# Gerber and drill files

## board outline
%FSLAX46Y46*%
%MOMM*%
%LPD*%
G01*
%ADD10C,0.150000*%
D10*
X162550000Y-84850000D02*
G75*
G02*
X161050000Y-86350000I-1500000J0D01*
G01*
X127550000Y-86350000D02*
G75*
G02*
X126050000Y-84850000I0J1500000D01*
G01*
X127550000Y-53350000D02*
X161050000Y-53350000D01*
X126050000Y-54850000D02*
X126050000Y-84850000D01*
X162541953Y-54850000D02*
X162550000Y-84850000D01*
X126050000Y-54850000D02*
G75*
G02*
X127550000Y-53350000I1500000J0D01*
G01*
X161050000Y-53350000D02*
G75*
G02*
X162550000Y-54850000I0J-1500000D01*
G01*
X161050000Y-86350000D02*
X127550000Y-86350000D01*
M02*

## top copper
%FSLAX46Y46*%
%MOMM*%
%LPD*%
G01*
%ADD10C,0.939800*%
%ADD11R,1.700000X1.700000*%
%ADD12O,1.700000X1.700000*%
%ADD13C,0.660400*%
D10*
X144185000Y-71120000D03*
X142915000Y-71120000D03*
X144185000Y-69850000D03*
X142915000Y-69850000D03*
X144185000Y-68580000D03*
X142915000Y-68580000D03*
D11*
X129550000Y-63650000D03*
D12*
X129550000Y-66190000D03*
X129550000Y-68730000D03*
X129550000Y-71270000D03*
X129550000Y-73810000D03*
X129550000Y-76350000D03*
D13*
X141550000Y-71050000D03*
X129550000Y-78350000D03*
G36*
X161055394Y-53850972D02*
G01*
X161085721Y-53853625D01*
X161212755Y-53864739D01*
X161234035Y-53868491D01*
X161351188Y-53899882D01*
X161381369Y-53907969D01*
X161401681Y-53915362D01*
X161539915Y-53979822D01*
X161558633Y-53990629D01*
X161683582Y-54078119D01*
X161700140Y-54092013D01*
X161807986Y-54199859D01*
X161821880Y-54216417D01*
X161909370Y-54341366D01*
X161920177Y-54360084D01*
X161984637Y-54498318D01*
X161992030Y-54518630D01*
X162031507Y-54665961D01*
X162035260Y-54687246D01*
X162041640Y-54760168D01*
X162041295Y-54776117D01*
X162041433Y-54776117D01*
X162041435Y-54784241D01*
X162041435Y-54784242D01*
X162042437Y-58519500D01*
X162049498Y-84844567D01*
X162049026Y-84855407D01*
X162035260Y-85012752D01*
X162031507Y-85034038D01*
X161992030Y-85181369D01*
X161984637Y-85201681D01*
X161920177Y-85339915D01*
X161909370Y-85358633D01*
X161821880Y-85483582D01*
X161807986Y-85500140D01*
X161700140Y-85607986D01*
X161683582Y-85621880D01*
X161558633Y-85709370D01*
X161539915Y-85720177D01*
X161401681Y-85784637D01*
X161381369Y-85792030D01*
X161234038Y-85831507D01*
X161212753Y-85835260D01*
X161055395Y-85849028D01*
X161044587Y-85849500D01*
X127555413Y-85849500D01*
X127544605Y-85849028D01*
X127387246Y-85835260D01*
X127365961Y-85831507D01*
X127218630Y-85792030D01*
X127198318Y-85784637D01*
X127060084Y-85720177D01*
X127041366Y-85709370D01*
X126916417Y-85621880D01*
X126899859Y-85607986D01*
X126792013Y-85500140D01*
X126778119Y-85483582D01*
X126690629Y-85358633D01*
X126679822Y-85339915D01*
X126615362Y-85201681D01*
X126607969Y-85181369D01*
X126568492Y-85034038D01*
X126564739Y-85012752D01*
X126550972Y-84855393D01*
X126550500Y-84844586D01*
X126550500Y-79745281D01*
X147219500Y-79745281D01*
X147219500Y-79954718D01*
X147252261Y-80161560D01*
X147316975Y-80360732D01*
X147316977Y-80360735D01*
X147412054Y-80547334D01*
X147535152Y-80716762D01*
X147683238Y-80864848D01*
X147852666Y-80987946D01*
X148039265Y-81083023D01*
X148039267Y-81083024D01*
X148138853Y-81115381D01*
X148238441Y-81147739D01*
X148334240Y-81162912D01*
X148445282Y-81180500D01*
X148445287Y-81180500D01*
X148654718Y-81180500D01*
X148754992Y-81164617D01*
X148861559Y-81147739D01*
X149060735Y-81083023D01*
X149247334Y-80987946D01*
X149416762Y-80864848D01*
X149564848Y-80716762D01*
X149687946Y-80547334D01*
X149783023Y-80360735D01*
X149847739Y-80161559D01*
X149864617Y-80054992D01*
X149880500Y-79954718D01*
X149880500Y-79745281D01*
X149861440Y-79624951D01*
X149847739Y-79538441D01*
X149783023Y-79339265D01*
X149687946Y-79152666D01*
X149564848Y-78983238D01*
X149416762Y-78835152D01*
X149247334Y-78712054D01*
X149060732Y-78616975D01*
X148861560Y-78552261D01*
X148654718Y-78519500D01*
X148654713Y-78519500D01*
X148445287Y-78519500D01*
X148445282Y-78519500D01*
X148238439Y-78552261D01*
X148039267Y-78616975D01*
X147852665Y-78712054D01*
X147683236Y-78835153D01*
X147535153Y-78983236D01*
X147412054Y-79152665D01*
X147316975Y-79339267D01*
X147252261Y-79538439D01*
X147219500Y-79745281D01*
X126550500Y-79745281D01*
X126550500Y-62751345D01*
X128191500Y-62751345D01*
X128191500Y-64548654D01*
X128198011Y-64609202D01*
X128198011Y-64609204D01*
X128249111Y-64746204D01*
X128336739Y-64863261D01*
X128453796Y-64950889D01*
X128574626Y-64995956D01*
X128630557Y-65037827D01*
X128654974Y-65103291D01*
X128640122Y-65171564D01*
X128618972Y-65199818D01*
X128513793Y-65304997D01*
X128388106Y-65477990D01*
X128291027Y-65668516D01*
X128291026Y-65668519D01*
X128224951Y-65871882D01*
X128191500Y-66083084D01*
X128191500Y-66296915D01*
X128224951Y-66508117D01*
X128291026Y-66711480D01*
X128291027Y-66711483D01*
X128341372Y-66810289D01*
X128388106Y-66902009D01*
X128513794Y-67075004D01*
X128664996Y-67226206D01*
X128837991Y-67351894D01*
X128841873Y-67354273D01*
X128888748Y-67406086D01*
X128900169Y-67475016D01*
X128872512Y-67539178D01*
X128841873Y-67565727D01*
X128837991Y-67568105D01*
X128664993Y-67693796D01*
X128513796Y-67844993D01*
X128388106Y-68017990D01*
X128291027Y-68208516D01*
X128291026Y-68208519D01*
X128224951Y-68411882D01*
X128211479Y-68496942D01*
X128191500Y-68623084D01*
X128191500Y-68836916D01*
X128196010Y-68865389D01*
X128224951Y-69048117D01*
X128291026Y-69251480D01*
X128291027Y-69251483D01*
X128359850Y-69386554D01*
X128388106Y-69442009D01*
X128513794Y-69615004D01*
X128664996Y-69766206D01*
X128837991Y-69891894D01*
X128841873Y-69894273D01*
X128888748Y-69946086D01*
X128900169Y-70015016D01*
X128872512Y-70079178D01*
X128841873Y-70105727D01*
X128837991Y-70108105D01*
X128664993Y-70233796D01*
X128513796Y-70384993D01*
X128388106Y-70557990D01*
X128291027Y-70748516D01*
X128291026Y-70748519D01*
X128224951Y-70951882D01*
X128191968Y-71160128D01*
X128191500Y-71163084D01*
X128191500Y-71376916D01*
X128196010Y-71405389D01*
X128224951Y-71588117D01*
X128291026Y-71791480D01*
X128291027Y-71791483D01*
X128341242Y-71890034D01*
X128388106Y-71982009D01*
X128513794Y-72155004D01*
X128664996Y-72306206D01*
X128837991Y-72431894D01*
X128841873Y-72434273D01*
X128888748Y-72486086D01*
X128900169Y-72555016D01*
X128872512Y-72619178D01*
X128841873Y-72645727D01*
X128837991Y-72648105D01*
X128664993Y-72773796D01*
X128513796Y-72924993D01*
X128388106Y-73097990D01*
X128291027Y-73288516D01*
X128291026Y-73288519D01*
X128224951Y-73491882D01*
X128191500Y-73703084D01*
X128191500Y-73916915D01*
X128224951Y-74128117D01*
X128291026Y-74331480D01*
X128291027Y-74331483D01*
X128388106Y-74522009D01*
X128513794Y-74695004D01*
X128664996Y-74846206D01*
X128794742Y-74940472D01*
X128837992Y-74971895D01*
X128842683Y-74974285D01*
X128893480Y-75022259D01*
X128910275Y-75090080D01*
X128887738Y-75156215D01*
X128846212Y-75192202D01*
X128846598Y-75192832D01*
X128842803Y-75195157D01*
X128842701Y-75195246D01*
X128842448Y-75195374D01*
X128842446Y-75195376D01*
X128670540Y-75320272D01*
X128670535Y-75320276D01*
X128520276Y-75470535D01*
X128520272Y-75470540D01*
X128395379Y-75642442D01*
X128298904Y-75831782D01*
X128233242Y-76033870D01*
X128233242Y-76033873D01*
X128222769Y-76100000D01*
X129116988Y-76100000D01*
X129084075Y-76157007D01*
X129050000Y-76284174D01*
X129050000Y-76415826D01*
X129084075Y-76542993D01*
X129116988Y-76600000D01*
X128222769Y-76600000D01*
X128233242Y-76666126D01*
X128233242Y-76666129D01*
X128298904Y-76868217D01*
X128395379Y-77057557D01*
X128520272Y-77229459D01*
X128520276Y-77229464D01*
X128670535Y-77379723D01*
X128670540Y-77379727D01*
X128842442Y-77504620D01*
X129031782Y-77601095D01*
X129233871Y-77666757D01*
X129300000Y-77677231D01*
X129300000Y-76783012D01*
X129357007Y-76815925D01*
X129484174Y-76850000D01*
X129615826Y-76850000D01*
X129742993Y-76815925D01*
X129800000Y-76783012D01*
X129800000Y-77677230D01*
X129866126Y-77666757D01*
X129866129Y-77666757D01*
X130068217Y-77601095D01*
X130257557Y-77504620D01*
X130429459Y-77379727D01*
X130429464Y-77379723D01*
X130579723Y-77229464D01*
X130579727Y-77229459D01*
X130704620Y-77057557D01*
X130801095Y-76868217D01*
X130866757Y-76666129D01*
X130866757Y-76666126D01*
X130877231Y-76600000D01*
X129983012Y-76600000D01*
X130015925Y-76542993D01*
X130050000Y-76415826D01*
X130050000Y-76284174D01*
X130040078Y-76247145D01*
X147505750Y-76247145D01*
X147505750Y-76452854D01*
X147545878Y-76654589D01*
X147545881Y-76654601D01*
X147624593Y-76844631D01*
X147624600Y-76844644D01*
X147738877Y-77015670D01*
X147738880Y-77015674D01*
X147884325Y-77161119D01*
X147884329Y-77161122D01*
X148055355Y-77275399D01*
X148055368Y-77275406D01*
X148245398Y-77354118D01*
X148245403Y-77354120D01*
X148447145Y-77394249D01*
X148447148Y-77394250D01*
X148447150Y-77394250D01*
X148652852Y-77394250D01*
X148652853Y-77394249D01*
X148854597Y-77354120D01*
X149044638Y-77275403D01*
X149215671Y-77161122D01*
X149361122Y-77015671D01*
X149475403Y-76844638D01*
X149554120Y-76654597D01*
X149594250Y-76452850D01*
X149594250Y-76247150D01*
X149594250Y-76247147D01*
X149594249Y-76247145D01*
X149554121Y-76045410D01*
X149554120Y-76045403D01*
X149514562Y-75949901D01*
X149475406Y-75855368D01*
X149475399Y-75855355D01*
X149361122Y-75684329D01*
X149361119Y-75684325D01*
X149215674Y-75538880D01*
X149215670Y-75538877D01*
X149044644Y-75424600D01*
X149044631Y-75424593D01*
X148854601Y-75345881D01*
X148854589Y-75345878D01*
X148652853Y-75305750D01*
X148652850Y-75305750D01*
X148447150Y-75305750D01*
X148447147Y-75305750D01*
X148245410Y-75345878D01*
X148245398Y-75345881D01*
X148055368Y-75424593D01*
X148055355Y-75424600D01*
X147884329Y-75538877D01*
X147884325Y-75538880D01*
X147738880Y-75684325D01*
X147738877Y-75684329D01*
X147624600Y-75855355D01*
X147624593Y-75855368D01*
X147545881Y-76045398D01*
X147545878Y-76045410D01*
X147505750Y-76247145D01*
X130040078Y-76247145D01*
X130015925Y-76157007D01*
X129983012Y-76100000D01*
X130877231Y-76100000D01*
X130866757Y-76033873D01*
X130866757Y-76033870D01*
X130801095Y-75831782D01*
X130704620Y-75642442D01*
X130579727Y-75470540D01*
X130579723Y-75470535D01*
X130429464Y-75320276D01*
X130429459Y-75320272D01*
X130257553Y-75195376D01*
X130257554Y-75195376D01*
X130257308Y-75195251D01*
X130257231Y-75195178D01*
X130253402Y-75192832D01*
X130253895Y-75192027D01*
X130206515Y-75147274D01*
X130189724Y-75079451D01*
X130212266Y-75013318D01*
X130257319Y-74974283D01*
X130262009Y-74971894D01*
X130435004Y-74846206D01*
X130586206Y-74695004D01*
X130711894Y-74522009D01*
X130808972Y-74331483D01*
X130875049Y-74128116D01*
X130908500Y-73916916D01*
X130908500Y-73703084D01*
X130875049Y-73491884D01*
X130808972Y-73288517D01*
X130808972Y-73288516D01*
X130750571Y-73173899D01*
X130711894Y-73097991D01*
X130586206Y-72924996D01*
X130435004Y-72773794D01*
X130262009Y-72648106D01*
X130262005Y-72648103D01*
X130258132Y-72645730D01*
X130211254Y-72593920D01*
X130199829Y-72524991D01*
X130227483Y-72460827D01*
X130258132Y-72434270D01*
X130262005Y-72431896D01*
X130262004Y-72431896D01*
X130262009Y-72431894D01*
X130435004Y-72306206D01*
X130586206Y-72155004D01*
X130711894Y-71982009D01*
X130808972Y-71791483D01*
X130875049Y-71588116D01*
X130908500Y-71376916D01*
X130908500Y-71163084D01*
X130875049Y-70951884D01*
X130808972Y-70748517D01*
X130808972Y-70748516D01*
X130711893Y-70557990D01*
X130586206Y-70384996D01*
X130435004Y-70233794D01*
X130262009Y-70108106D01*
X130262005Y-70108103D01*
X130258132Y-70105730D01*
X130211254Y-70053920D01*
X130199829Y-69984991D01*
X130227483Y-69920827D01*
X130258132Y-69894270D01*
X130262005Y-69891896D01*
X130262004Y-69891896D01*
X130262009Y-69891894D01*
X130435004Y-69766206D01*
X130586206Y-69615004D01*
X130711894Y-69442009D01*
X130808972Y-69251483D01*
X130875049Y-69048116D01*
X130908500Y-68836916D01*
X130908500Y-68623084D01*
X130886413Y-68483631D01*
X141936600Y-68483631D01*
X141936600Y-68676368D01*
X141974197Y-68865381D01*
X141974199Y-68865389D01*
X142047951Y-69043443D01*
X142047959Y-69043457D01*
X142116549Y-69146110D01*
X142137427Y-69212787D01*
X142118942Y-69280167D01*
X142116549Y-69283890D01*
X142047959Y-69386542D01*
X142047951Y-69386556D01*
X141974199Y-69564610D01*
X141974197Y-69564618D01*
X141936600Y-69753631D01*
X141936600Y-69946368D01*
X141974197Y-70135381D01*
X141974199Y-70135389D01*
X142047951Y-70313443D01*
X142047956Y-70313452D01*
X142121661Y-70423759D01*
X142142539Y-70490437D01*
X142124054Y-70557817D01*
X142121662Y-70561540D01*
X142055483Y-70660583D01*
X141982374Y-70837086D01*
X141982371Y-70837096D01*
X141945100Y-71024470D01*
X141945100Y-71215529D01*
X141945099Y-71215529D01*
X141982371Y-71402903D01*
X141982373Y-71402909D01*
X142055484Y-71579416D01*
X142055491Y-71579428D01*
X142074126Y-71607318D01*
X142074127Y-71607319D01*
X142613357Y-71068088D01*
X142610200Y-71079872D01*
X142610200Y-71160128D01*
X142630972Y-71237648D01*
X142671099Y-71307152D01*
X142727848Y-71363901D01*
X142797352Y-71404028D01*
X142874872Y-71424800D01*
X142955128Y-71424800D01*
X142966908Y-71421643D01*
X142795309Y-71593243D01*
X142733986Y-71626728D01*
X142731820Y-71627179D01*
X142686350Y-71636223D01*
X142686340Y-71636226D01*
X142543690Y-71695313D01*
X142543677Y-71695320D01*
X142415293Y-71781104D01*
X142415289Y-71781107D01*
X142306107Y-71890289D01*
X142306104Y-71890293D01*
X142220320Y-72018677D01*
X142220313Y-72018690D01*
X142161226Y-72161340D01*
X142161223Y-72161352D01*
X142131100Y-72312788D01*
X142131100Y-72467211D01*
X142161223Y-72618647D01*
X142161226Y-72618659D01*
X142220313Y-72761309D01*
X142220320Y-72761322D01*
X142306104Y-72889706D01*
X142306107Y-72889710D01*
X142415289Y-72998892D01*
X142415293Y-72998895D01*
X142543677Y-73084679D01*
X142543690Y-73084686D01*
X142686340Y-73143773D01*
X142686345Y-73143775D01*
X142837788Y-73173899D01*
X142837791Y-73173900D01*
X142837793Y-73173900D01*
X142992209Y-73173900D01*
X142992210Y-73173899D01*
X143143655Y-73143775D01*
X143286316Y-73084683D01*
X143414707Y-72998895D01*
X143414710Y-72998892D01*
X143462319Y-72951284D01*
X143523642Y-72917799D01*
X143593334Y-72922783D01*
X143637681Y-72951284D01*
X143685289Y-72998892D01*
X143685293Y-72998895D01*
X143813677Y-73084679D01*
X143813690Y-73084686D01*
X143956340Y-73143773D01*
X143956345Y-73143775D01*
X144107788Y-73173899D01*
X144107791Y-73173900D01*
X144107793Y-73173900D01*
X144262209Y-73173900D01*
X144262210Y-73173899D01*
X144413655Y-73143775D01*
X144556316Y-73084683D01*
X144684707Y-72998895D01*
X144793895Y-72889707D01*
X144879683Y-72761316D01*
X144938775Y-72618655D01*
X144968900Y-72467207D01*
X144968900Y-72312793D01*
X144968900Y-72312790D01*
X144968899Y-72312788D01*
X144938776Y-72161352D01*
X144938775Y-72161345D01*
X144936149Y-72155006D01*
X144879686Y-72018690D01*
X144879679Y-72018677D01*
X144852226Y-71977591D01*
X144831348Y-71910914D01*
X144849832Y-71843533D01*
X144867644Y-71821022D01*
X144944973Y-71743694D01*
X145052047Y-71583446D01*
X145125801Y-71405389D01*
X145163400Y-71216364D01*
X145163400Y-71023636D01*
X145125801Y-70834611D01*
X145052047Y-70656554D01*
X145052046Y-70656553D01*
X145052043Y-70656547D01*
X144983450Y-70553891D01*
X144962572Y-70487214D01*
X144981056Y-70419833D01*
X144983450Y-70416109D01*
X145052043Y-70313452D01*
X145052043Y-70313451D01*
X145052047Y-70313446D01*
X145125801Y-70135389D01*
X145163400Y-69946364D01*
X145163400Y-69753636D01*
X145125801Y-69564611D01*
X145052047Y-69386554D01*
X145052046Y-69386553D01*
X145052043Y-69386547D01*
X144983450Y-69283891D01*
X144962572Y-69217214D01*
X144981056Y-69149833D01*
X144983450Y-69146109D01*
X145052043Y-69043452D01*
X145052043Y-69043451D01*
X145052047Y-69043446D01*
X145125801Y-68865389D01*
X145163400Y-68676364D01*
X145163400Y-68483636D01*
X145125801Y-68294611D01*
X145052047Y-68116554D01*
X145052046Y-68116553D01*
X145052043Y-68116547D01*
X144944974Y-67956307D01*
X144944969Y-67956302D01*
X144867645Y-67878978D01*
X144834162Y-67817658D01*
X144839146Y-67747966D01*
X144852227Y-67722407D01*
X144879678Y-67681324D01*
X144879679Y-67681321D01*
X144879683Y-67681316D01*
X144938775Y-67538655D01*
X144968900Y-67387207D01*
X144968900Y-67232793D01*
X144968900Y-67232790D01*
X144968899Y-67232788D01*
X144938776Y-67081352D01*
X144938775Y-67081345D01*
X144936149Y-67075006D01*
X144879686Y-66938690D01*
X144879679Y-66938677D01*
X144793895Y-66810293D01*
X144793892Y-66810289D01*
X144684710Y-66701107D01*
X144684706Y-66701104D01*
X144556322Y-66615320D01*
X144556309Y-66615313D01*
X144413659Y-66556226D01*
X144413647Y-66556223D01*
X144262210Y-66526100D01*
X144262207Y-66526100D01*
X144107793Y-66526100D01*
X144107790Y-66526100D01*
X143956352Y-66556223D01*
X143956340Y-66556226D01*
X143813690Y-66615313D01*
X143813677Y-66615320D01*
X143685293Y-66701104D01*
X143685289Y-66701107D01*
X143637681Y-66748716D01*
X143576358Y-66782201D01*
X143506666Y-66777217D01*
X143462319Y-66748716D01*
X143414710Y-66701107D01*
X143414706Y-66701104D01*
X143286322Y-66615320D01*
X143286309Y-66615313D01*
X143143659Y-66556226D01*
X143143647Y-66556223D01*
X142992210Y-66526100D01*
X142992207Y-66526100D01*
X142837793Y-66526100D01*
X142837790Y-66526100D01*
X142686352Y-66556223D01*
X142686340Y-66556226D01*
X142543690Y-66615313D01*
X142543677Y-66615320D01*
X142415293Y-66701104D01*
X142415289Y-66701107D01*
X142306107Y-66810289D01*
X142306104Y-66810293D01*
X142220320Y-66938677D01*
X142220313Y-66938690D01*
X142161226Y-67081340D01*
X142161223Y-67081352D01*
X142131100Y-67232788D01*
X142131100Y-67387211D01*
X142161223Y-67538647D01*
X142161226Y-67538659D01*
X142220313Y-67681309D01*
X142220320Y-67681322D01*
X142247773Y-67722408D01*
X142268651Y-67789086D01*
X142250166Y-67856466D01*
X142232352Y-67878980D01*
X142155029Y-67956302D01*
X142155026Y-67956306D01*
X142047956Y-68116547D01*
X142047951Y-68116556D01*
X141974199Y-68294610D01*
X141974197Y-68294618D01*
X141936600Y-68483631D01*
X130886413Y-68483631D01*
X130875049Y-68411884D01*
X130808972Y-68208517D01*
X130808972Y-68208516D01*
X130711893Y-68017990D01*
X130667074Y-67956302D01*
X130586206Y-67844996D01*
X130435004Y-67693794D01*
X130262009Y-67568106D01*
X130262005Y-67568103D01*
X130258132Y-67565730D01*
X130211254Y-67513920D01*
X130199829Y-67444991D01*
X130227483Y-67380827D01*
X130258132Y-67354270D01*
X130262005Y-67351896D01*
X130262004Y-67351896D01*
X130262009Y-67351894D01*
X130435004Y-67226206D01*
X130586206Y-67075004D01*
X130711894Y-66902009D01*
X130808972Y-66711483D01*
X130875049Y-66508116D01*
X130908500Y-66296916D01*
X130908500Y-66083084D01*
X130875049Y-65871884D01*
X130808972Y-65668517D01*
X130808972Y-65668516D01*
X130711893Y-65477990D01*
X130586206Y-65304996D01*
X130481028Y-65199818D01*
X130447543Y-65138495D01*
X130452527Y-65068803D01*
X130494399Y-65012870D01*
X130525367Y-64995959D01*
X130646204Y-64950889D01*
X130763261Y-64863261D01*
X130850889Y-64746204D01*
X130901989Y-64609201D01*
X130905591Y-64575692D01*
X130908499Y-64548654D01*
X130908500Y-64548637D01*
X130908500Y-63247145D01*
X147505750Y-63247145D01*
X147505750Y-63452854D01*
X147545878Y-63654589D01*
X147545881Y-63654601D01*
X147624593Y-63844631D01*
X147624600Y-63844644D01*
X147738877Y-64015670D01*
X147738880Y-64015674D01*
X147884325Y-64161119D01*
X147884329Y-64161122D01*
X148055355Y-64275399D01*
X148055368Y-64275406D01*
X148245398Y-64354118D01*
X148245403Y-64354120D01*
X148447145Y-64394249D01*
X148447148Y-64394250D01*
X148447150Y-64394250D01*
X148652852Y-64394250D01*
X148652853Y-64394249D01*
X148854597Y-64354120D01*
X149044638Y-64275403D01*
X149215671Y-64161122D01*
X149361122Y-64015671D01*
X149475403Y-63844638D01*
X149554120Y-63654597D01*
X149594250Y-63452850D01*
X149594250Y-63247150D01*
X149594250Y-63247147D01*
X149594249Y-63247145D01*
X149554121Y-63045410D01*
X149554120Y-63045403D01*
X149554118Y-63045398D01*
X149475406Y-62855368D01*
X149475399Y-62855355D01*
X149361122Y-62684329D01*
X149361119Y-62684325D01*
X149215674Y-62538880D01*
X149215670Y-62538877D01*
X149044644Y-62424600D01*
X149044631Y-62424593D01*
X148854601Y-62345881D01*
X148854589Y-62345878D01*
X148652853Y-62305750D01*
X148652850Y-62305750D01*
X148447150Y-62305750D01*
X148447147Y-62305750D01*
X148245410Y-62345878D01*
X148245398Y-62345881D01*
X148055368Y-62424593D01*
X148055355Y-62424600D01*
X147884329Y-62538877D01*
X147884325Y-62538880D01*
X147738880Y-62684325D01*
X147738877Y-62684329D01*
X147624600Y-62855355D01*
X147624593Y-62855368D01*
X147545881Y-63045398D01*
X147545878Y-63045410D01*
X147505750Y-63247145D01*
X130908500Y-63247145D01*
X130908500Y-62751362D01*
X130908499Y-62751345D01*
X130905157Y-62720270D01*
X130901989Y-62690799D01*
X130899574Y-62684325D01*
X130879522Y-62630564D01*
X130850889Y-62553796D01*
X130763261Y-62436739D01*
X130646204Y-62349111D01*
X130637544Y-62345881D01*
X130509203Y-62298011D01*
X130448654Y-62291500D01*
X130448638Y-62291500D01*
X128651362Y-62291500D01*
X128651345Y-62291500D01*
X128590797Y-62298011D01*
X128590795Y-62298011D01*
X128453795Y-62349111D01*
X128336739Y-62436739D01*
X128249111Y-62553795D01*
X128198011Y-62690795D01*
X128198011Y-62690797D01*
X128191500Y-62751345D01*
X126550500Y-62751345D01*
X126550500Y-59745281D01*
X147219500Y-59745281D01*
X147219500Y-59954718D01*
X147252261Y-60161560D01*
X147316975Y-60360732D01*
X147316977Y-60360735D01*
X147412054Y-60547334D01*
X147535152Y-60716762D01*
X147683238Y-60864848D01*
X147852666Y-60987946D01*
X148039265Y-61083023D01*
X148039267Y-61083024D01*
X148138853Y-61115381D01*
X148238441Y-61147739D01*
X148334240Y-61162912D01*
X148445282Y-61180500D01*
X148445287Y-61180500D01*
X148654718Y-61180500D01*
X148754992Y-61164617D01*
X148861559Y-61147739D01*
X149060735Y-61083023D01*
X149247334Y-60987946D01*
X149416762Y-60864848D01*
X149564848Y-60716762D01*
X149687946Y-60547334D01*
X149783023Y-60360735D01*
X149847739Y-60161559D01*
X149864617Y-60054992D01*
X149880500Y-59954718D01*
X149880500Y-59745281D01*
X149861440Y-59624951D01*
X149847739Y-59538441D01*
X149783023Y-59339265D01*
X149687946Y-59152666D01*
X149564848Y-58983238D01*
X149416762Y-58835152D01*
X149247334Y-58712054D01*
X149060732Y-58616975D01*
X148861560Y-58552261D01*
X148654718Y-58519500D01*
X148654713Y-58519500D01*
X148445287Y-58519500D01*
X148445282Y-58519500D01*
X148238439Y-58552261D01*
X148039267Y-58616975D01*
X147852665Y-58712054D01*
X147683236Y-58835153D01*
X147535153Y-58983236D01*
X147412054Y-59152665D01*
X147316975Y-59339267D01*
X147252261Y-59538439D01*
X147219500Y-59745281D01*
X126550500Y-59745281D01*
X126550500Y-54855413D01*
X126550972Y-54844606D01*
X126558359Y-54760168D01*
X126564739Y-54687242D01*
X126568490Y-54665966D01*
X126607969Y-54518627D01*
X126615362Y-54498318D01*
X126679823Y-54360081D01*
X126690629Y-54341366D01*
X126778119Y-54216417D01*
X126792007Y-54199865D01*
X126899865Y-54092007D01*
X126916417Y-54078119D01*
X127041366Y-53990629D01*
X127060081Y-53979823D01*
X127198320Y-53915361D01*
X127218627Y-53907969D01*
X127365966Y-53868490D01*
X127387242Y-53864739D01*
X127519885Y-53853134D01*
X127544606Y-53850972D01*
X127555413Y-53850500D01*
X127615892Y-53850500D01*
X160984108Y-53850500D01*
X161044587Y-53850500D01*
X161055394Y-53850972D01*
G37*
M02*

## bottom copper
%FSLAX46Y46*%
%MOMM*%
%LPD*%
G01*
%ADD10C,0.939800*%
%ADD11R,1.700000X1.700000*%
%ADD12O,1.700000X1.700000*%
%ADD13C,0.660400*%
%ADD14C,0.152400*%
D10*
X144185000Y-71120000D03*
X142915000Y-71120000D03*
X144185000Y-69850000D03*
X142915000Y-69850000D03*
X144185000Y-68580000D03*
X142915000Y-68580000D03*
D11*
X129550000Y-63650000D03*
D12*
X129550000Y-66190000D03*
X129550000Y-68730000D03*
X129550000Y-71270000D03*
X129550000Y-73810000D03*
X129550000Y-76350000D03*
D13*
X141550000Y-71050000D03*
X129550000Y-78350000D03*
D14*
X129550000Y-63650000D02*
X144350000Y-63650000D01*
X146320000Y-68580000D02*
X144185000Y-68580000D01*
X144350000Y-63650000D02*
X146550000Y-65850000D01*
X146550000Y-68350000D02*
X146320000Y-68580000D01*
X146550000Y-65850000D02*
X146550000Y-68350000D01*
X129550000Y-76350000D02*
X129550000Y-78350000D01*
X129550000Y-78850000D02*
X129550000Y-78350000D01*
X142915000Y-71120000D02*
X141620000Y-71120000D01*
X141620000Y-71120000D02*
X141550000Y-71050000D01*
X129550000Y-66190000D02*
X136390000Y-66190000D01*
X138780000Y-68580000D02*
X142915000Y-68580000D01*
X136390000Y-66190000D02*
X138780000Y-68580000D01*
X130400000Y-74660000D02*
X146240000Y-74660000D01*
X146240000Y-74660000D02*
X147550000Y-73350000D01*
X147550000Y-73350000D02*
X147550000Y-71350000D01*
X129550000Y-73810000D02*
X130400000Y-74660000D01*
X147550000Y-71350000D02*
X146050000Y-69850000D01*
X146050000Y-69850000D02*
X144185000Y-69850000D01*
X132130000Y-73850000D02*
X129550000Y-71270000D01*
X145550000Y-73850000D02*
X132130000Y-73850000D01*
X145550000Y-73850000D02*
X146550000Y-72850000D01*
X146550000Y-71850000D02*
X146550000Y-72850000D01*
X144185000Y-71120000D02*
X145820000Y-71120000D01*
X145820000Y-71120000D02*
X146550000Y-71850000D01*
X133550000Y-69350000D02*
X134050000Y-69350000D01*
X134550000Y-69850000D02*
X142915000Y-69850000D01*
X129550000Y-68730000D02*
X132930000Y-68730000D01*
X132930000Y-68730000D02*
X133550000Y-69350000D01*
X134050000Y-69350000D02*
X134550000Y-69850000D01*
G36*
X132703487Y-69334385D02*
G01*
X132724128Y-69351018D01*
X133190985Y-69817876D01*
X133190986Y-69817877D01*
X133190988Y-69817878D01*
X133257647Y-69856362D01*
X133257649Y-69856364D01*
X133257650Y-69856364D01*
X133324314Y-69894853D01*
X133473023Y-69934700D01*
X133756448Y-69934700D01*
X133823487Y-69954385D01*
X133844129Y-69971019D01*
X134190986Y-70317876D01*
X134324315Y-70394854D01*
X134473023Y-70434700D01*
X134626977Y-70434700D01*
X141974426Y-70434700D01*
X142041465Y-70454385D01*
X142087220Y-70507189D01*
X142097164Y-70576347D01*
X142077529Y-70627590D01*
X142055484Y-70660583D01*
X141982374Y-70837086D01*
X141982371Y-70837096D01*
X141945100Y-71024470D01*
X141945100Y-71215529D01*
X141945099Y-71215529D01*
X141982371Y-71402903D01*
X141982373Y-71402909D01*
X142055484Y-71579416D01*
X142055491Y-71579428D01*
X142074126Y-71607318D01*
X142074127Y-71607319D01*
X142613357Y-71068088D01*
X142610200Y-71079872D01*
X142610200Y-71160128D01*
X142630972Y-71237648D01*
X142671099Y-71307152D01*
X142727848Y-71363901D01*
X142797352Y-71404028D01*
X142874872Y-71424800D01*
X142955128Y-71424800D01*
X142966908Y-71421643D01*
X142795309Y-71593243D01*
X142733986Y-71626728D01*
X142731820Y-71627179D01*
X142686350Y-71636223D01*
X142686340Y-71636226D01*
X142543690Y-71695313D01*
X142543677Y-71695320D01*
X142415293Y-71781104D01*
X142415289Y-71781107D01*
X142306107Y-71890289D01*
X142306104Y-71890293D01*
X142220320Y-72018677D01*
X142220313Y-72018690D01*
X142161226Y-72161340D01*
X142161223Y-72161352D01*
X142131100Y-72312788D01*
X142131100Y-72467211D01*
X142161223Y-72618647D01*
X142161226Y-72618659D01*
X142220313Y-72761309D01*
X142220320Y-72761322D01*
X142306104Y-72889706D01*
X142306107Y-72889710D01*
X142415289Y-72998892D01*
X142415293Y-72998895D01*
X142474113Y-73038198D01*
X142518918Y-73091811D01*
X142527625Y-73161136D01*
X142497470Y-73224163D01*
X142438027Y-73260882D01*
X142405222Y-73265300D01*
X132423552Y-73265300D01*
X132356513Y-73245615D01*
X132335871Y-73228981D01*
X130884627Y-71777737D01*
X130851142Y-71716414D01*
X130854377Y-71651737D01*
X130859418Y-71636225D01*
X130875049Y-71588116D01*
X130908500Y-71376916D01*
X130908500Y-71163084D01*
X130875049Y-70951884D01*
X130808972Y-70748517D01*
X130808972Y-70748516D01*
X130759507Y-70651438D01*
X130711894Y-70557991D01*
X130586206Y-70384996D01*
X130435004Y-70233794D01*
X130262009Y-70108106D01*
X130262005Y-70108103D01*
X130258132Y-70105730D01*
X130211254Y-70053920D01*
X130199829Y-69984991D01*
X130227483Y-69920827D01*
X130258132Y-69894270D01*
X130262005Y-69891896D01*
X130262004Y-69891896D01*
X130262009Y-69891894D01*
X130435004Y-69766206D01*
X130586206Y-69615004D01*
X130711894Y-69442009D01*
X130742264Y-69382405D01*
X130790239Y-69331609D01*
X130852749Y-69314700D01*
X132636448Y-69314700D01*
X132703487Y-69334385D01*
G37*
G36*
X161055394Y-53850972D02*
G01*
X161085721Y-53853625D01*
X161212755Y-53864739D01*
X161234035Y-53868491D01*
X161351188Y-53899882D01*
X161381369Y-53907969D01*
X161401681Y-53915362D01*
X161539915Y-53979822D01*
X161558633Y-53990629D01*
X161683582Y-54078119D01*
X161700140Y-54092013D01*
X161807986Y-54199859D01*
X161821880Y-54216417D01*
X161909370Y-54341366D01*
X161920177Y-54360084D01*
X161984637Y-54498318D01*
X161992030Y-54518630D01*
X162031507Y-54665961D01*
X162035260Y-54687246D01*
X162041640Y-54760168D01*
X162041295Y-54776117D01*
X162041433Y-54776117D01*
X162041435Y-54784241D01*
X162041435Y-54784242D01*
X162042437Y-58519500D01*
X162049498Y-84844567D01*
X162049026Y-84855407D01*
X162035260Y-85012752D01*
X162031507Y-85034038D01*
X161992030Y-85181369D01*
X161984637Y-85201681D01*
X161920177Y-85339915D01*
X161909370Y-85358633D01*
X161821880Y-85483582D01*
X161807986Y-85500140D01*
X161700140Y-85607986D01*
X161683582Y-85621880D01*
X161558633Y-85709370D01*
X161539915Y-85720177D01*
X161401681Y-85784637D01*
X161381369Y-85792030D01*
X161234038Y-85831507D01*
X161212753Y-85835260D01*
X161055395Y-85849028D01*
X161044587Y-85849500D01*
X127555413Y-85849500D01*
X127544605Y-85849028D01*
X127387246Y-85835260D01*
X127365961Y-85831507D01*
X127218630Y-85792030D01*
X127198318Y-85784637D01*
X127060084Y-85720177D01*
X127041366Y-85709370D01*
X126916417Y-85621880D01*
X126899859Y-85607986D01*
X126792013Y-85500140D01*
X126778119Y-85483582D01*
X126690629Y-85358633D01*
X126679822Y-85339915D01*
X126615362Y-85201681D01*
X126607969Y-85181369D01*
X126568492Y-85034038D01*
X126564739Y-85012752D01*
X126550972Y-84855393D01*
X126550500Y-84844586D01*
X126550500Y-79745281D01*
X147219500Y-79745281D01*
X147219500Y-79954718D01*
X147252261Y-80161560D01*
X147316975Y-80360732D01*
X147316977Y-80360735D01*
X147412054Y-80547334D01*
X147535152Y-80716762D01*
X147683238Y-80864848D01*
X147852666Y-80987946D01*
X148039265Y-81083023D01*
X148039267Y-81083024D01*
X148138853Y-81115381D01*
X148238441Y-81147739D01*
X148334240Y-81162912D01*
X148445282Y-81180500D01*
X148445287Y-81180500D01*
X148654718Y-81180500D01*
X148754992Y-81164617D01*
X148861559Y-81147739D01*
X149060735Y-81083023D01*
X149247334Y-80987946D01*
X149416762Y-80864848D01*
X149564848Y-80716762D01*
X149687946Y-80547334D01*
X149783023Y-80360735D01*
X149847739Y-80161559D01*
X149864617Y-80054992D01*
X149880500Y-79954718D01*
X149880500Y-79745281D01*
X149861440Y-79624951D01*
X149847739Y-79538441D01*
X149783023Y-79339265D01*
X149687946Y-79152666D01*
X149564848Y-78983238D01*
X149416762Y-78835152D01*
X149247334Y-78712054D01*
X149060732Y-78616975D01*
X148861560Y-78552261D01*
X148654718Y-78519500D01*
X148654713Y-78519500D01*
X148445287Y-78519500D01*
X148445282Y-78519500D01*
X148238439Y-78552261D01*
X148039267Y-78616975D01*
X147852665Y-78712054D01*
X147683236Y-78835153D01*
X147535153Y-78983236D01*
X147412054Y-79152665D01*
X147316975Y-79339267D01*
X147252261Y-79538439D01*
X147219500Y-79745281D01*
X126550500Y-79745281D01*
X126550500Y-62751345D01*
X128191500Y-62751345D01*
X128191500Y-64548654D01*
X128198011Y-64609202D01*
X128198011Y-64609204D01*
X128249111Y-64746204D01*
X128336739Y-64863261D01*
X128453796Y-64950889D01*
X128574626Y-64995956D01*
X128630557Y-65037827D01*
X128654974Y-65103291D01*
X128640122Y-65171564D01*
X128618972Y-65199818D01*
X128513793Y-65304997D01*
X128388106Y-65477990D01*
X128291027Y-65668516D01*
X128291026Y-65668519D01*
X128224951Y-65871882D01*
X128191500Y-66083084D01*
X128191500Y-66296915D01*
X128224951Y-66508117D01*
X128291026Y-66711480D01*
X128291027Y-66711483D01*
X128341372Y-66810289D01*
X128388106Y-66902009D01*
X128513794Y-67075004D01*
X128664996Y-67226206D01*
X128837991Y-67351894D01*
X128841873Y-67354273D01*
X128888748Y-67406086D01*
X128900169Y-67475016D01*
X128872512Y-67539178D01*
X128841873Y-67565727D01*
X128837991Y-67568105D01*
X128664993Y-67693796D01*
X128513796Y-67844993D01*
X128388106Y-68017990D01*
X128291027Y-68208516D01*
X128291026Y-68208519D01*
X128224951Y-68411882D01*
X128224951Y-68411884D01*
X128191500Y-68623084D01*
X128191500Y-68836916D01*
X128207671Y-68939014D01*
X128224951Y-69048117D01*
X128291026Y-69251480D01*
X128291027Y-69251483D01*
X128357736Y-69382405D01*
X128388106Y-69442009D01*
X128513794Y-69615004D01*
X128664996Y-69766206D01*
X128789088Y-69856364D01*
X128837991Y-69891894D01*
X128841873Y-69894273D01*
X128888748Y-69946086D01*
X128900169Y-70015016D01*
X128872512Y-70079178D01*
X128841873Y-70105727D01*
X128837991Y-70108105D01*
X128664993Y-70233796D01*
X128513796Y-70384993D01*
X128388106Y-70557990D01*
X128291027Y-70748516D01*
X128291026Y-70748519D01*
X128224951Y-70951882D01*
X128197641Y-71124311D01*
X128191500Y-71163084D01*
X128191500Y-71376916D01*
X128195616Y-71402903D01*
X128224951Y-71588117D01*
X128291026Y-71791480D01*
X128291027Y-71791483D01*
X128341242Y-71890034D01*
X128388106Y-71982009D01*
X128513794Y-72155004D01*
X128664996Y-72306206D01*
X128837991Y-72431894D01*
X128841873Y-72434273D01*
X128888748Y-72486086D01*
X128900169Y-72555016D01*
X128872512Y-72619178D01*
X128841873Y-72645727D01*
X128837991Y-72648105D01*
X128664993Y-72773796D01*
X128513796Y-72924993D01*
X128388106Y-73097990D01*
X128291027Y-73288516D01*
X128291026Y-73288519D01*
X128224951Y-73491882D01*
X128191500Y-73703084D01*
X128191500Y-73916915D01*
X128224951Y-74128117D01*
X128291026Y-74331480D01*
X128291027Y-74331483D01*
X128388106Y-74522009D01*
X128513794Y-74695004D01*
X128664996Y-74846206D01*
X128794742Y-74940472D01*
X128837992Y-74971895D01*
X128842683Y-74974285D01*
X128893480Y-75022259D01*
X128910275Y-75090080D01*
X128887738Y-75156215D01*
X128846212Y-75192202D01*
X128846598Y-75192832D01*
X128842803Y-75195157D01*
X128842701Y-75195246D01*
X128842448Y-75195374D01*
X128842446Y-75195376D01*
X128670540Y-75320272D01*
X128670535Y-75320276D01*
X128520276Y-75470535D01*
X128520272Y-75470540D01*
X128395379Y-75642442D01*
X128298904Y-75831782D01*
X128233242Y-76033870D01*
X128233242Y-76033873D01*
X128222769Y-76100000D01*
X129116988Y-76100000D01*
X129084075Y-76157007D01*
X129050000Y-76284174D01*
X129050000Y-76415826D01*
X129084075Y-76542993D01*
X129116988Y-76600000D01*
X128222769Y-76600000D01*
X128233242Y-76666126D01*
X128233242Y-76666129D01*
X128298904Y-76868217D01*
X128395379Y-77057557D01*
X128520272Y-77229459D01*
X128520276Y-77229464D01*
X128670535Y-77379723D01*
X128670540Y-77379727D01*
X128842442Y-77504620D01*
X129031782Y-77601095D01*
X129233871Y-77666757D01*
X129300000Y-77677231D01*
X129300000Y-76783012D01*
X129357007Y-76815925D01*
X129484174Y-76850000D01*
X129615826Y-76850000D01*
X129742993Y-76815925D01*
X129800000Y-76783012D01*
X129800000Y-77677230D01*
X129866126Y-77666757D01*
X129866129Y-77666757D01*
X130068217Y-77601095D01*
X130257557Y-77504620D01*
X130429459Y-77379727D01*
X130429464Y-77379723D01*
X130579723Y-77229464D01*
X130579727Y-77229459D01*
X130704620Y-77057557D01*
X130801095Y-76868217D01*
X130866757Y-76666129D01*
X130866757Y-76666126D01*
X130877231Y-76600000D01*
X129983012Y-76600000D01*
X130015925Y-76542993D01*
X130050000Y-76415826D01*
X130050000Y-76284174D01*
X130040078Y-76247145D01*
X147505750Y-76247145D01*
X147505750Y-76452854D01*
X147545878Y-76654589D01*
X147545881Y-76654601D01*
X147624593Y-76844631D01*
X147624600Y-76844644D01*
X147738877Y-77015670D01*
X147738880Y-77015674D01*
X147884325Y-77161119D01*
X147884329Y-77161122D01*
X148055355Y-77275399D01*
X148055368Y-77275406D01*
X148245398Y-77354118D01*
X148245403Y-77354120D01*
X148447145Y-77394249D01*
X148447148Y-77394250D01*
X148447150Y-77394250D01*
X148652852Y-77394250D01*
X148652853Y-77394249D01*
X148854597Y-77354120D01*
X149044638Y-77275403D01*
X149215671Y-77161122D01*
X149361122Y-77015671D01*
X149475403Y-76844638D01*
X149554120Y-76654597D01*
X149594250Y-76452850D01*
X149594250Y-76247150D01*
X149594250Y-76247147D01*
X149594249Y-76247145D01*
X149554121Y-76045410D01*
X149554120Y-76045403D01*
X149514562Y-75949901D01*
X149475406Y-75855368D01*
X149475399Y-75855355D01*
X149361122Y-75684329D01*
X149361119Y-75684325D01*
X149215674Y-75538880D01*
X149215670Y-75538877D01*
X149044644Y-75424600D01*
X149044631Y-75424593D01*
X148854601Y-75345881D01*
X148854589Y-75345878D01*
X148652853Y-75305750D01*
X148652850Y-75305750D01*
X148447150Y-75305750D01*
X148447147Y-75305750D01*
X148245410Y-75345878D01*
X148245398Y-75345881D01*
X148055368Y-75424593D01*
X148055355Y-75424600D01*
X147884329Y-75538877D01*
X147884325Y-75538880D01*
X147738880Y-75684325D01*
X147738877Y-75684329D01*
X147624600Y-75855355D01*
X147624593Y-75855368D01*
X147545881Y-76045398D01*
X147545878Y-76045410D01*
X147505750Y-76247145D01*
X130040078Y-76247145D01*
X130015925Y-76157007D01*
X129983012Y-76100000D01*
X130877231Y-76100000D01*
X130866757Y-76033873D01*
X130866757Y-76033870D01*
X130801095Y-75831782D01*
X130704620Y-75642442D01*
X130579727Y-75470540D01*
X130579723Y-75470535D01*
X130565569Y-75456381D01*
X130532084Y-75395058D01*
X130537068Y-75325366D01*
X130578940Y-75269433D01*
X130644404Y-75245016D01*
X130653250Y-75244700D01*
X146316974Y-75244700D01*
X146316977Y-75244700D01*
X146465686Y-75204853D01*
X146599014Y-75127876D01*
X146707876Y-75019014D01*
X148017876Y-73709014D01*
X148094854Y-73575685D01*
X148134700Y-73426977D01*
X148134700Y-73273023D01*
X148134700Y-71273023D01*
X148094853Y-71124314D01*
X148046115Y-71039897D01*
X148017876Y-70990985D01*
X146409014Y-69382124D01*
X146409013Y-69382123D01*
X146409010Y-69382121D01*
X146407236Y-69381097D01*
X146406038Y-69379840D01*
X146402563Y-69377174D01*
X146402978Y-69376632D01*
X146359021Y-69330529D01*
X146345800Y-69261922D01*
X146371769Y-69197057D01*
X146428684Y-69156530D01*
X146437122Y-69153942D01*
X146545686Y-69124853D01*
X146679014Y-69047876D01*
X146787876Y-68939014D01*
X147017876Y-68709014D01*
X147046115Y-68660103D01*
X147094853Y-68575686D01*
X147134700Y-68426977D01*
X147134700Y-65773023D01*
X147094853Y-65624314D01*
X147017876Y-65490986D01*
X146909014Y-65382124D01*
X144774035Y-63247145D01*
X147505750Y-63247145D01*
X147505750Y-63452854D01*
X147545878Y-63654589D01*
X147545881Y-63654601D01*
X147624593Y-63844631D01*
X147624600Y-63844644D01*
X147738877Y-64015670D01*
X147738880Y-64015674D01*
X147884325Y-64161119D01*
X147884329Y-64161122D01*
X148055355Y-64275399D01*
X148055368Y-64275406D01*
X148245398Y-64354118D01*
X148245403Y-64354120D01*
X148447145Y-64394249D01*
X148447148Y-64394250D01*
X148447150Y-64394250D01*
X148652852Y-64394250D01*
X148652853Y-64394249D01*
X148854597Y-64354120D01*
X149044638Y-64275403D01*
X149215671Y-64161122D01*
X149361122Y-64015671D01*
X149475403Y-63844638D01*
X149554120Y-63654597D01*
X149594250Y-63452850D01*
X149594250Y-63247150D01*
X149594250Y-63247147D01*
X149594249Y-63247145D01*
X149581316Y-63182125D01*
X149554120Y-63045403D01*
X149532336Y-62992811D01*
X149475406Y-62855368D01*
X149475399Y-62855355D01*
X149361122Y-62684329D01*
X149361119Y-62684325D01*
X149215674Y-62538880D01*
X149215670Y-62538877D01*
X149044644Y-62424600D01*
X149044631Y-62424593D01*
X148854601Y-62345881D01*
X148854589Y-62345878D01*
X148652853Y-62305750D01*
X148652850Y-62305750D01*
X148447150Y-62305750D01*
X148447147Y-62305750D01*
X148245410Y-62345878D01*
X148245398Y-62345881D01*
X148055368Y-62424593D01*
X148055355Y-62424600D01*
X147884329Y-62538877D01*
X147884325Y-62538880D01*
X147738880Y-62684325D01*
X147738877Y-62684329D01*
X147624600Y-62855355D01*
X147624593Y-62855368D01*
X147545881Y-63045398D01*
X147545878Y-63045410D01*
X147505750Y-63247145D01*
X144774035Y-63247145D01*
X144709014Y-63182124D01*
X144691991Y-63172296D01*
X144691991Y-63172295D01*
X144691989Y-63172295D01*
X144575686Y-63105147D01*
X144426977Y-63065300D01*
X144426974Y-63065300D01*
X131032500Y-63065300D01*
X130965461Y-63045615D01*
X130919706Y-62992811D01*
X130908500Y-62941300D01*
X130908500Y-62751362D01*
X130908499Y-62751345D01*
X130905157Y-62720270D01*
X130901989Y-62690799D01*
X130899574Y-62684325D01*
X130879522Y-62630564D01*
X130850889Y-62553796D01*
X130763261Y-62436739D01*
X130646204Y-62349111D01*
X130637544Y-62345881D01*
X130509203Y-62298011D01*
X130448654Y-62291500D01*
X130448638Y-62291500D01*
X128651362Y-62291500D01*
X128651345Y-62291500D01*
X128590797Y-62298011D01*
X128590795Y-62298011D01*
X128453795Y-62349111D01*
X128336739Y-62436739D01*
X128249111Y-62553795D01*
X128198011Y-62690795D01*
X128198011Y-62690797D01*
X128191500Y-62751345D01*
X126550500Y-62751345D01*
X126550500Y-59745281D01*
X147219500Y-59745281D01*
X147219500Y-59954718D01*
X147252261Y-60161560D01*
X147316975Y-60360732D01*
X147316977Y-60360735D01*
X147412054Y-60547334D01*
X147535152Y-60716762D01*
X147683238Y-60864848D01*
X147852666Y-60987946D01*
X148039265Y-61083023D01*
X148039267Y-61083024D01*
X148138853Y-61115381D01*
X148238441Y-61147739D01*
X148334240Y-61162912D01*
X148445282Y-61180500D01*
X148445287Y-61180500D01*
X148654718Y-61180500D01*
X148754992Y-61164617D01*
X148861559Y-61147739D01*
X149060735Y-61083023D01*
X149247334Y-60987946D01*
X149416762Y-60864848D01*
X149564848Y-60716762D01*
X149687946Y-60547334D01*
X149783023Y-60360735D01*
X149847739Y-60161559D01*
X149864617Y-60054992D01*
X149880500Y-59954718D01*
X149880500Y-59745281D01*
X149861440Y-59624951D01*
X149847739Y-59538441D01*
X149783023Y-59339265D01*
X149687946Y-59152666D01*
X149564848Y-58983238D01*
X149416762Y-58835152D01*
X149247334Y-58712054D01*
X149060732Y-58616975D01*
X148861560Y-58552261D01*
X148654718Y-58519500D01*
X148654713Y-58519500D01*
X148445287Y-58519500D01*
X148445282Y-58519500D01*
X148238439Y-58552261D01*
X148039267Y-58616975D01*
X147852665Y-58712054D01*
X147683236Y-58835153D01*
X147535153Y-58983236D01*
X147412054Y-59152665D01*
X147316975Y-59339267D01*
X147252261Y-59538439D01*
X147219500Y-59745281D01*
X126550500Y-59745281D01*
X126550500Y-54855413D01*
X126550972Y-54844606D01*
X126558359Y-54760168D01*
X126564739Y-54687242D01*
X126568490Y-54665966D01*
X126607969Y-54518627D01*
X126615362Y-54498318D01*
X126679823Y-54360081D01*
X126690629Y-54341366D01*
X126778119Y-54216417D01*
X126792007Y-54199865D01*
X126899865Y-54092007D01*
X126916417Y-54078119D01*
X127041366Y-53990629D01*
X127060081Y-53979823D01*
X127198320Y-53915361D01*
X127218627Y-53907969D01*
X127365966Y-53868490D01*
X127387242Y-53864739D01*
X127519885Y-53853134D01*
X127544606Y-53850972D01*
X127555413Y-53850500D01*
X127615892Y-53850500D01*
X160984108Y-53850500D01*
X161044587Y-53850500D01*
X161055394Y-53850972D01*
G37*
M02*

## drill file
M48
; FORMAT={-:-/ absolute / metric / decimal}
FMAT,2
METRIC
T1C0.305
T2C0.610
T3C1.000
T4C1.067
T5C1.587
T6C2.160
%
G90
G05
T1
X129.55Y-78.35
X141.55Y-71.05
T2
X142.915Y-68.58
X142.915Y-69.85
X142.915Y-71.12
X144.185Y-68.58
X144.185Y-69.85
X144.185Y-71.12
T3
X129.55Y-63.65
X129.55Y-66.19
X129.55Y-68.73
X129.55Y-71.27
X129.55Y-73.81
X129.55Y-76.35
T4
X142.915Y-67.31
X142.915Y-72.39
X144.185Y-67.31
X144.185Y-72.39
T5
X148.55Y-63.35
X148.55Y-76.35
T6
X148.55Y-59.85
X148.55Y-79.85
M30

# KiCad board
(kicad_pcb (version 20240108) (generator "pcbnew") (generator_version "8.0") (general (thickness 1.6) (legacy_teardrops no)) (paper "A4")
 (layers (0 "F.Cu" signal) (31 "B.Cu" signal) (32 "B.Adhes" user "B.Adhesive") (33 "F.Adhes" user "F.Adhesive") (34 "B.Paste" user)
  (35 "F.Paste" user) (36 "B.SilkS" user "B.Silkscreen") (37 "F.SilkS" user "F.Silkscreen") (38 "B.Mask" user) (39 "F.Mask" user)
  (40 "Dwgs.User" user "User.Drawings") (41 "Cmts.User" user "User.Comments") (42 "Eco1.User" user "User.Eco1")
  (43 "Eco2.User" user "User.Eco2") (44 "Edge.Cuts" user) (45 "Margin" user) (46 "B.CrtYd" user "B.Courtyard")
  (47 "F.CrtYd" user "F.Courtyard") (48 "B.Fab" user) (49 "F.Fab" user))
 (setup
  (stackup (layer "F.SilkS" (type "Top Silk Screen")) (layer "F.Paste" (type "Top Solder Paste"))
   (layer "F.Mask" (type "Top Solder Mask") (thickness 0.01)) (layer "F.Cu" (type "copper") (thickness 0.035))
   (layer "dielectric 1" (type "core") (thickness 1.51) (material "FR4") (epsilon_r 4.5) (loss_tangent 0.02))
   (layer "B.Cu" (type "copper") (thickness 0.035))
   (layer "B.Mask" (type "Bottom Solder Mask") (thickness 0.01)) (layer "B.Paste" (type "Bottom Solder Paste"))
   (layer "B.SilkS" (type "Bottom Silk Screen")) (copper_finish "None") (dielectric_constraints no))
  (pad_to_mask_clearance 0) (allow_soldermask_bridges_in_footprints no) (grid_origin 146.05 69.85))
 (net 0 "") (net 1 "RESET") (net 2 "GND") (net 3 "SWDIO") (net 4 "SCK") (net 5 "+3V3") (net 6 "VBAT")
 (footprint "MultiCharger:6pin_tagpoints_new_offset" (layer "F.Cu") (at 143.55 69.85 90)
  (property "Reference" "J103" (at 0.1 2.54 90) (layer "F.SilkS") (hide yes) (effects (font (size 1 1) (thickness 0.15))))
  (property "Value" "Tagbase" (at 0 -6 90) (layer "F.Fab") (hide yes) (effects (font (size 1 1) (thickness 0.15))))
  (pad "" np_thru_hole circle (at -10 5 90) (size 2.16 2.16) (drill 2.16) (layers "*.Cu" "*.Mask"))
  (pad "" np_thru_hole circle (at -6.5 5 90) (size 1.5875 1.5875) (drill 1.5875) (layers "*.Cu" "*.Mask"))
  (pad "" np_thru_hole circle (at -2.54 -0.635 90) (size 1.0668 1.0668) (drill 1.0668) (layers "*.Cu"))
  (pad "" np_thru_hole circle (at -2.54 0.635 90) (size 1.0668 1.0668) (drill 1.0668) (layers "*.Cu"))
  (pad "" np_thru_hole circle (at 2.54 -0.635 90) (size 1.0668 1.0668) (drill 1.0668) (layers "*.Cu"))
  (pad "" np_thru_hole circle (at 2.54 0.635 90) (size 1.0668 1.0668) (drill 1.0668) (layers "*.Cu"))
  (pad "" np_thru_hole circle (at 6.5 5 90) (size 1.5875 1.5875) (drill 1.5875) (layers "*.Cu" "*.Mask"))
  (pad "" np_thru_hole circle (at 10 5 90) (size 2.16 2.16) (drill 2.16) (layers "*.Cu" "*.Mask"))
  (pad "1" thru_hole circle (at -1.27 0.635 90) (size 0.9398 0.9398) (drill 0.6096) (layers "*.Cu" "*.Mask") (remove_unused_layers no)
   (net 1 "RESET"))
  (pad "2" thru_hole circle (at -1.27 -0.635 90) (size 0.9398 0.9398) (drill 0.6096) (layers "*.Cu" "*.Mask") (remove_unused_layers no)
   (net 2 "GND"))
  (pad "3" thru_hole circle (at 0 0.635 90) (size 0.9398 0.9398) (drill 0.6096) (layers "*.Cu" "*.Mask") (remove_unused_layers no)
   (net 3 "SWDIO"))
  (pad "4" thru_hole circle (at 0 -0.635 90) (size 0.9398 0.9398) (drill 0.6096) (layers "*.Cu" "*.Mask") (remove_unused_layers no)
   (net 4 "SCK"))
  (pad "5" thru_hole circle (at 1.27 0.635 90) (size 0.9398 0.9398) (drill 0.6096) (layers "*.Cu" "*.Mask") (remove_unused_layers no)
   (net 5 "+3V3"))
  (pad "6" thru_hole circle (at 1.27 -0.635 90) (size 0.9398 0.9398) (drill 0.6096) (layers "*.Cu" "*.Mask") (remove_unused_layers no)
   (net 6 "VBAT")))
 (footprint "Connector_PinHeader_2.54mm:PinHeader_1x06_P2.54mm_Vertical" (layer "F.Cu") (at 129.55 63.65)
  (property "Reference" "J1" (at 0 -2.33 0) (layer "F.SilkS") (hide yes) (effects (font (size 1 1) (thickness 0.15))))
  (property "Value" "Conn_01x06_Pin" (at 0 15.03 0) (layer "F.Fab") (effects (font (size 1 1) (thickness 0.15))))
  (pad "1" thru_hole rect (at 0 0) (size 1.7 1.7) (drill 1) (layers "*.Cu" "*.Mask") (remove_unused_layers no) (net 5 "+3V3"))
  (pad "2" thru_hole oval (at 0 2.54) (size 1.7 1.7) (drill 1) (layers "*.Cu" "*.Mask") (remove_unused_layers no) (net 6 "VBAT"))
  (pad "3" thru_hole oval (at 0 5.08) (size 1.7 1.7) (drill 1) (layers "*.Cu" "*.Mask") (remove_unused_layers no) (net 4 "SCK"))
  (pad "4" thru_hole oval (at 0 7.62) (size 1.7 1.7) (drill 1) (layers "*.Cu" "*.Mask") (remove_unused_layers no) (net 1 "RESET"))
  (pad "5" thru_hole oval (at 0 10.16) (size 1.7 1.7) (drill 1) (layers "*.Cu" "*.Mask") (remove_unused_layers no) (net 3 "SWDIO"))
  (pad "6" thru_hole oval (at 0 12.7) (size 1.7 1.7) (drill 1) (layers "*.Cu" "*.Mask") (remove_unused_layers no) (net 2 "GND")))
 (gr_arc (start 162.55 84.85) (mid 162.11066 85.91066) (end 161.05 86.35) (stroke (width 0.15) (type default)) (layer "Edge.Cuts"))
 (gr_arc (start 127.55 86.35) (mid 126.48934 85.91066) (end 126.05 84.85) (stroke (width 0.15) (type default)) (layer "Edge.Cuts"))
 (gr_line (start 127.55 53.35) (end 161.05 53.35) (stroke (width 0.15) (type solid)) (layer "Edge.Cuts"))
 (gr_line (start 126.05 54.85) (end 126.05 84.85) (stroke (width 0.15) (type default)) (layer "Edge.Cuts"))
 (gr_line (start 162.541953 54.85) (end 162.55 84.85) (stroke (width 0.15) (type default)) (layer "Edge.Cuts"))
 (gr_arc (start 126.05 54.85) (mid 126.48934 53.78934) (end 127.55 53.35) (stroke (width 0.15) (type default)) (layer "Edge.Cuts"))
 (gr_arc (start 161.05 53.35) (mid 162.11066 53.78934) (end 162.55 54.85) (stroke (width 0.15) (type default)) (layer "Edge.Cuts"))
 (gr_line (start 161.05 86.35) (end 127.55 86.35) (stroke (width 0.15) (type solid)) (layer "Edge.Cuts"))
 (segment (start 129.55 63.65) (end 144.35 63.65) (width 0.1524) (layer "B.Cu") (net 5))
 (segment (start 146.32 68.58) (end 144.185 68.58) (width 0.1524) (layer "B.Cu") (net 5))
 (segment (start 144.35 63.65) (end 146.55 65.85) (width 0.1524) (layer "B.Cu") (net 5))
 (segment (start 146.55 68.35) (end 146.32 68.58) (width 0.1524) (layer "B.Cu") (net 5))
 (segment (start 146.55 65.85) (end 146.55 68.35) (width 0.1524) (layer "B.Cu") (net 5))
 (via (at 141.55 71.05) (size 0.6604) (drill 0.3048) (layers "F.Cu" "B.Cu") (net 2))
 (via (at 129.55 78.35) (size 0.6604) (drill 0.3048) (layers "F.Cu" "B.Cu") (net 2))
 (segment (start 129.55 76.35) (end 129.55 78.35) (width 0.1524) (layer "B.Cu") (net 2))
 (segment (start 129.55 78.85) (end 129.55 78.35) (width 0.1524) (layer "B.Cu") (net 2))
 (segment (start 142.915 71.12) (end 141.62 71.12) (width 0.1524) (layer "B.Cu") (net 2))
 (segment (start 141.62 71.12) (end 141.55 71.05) (width 0.1524) (layer "B.Cu") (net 2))
 (segment (start 129.55 66.19) (end 136.39 66.19) (width 0.1524) (layer "B.Cu") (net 6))
 (segment (start 138.78 68.58) (end 142.915 68.58) (width 0.1524) (layer "B.Cu") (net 6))
 (segment (start 136.39 66.19) (end 138.78 68.58) (width 0.1524) (layer "B.Cu") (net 6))
 (segment (start 130.4 74.66) (end 146.24 74.66) (width 0.1524) (layer "B.Cu") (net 3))
 (segment (start 146.24 74.66) (end 147.55 73.35) (width 0.1524) (layer "B.Cu") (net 3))
 (segment (start 147.55 73.35) (end 147.55 71.35) (width 0.1524) (layer "B.Cu") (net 3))
 (segment (start 129.55 73.81) (end 130.4 74.66) (width 0.1524) (layer "B.Cu") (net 3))
 (segment (start 147.55 71.35) (end 146.05 69.85) (width 0.1524) (layer "B.Cu") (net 3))
 (segment (start 146.05 69.85) (end 144.185 69.85) (width 0.1524) (layer "B.Cu") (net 3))
 (segment (start 132.13 73.85) (end 129.55 71.27) (width 0.1524) (layer "B.Cu") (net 1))
 (segment (start 145.55 73.85) (end 132.13 73.85) (width 0.1524) (layer "B.Cu") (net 1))
 (segment (start 145.55 73.85) (end 146.55 72.85) (width 0.1524) (layer "B.Cu") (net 1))
 (segment (start 146.55 71.85) (end 146.55 72.85) (width 0.1524) (layer "B.Cu") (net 1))
 (segment (start 144.185 71.12) (end 145.82 71.12) (width 0.1524) (layer "B.Cu") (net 1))
 (segment (start 145.82 71.12) (end 146.55 71.85) (width 0.1524) (layer "B.Cu") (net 1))
 (segment (start 133.55 69.35) (end 134.05 69.35) (width 0.1524) (layer "B.Cu") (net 4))
 (segment (start 134.55 69.85) (end 142.915 69.85) (width 0.1524) (layer "B.Cu") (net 4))
 (segment (start 129.55 68.73) (end 132.93 68.73) (width 0.1524) (layer "B.Cu") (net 4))
 (segment (start 132.93 68.73) (end 133.55 69.35) (width 0.1524) (layer "B.Cu") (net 4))
 (segment (start 134.05 69.35) (end 134.55 69.85) (width 0.1524) (layer "B.Cu") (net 4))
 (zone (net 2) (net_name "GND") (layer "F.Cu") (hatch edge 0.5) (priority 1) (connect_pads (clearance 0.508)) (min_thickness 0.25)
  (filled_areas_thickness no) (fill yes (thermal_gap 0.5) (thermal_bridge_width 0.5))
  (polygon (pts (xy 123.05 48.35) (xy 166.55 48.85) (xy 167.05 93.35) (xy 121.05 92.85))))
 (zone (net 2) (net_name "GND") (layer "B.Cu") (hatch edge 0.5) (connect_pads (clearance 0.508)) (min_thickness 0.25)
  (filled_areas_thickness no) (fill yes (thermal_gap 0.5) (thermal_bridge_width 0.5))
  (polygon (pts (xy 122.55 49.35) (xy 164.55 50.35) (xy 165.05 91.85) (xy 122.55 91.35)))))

